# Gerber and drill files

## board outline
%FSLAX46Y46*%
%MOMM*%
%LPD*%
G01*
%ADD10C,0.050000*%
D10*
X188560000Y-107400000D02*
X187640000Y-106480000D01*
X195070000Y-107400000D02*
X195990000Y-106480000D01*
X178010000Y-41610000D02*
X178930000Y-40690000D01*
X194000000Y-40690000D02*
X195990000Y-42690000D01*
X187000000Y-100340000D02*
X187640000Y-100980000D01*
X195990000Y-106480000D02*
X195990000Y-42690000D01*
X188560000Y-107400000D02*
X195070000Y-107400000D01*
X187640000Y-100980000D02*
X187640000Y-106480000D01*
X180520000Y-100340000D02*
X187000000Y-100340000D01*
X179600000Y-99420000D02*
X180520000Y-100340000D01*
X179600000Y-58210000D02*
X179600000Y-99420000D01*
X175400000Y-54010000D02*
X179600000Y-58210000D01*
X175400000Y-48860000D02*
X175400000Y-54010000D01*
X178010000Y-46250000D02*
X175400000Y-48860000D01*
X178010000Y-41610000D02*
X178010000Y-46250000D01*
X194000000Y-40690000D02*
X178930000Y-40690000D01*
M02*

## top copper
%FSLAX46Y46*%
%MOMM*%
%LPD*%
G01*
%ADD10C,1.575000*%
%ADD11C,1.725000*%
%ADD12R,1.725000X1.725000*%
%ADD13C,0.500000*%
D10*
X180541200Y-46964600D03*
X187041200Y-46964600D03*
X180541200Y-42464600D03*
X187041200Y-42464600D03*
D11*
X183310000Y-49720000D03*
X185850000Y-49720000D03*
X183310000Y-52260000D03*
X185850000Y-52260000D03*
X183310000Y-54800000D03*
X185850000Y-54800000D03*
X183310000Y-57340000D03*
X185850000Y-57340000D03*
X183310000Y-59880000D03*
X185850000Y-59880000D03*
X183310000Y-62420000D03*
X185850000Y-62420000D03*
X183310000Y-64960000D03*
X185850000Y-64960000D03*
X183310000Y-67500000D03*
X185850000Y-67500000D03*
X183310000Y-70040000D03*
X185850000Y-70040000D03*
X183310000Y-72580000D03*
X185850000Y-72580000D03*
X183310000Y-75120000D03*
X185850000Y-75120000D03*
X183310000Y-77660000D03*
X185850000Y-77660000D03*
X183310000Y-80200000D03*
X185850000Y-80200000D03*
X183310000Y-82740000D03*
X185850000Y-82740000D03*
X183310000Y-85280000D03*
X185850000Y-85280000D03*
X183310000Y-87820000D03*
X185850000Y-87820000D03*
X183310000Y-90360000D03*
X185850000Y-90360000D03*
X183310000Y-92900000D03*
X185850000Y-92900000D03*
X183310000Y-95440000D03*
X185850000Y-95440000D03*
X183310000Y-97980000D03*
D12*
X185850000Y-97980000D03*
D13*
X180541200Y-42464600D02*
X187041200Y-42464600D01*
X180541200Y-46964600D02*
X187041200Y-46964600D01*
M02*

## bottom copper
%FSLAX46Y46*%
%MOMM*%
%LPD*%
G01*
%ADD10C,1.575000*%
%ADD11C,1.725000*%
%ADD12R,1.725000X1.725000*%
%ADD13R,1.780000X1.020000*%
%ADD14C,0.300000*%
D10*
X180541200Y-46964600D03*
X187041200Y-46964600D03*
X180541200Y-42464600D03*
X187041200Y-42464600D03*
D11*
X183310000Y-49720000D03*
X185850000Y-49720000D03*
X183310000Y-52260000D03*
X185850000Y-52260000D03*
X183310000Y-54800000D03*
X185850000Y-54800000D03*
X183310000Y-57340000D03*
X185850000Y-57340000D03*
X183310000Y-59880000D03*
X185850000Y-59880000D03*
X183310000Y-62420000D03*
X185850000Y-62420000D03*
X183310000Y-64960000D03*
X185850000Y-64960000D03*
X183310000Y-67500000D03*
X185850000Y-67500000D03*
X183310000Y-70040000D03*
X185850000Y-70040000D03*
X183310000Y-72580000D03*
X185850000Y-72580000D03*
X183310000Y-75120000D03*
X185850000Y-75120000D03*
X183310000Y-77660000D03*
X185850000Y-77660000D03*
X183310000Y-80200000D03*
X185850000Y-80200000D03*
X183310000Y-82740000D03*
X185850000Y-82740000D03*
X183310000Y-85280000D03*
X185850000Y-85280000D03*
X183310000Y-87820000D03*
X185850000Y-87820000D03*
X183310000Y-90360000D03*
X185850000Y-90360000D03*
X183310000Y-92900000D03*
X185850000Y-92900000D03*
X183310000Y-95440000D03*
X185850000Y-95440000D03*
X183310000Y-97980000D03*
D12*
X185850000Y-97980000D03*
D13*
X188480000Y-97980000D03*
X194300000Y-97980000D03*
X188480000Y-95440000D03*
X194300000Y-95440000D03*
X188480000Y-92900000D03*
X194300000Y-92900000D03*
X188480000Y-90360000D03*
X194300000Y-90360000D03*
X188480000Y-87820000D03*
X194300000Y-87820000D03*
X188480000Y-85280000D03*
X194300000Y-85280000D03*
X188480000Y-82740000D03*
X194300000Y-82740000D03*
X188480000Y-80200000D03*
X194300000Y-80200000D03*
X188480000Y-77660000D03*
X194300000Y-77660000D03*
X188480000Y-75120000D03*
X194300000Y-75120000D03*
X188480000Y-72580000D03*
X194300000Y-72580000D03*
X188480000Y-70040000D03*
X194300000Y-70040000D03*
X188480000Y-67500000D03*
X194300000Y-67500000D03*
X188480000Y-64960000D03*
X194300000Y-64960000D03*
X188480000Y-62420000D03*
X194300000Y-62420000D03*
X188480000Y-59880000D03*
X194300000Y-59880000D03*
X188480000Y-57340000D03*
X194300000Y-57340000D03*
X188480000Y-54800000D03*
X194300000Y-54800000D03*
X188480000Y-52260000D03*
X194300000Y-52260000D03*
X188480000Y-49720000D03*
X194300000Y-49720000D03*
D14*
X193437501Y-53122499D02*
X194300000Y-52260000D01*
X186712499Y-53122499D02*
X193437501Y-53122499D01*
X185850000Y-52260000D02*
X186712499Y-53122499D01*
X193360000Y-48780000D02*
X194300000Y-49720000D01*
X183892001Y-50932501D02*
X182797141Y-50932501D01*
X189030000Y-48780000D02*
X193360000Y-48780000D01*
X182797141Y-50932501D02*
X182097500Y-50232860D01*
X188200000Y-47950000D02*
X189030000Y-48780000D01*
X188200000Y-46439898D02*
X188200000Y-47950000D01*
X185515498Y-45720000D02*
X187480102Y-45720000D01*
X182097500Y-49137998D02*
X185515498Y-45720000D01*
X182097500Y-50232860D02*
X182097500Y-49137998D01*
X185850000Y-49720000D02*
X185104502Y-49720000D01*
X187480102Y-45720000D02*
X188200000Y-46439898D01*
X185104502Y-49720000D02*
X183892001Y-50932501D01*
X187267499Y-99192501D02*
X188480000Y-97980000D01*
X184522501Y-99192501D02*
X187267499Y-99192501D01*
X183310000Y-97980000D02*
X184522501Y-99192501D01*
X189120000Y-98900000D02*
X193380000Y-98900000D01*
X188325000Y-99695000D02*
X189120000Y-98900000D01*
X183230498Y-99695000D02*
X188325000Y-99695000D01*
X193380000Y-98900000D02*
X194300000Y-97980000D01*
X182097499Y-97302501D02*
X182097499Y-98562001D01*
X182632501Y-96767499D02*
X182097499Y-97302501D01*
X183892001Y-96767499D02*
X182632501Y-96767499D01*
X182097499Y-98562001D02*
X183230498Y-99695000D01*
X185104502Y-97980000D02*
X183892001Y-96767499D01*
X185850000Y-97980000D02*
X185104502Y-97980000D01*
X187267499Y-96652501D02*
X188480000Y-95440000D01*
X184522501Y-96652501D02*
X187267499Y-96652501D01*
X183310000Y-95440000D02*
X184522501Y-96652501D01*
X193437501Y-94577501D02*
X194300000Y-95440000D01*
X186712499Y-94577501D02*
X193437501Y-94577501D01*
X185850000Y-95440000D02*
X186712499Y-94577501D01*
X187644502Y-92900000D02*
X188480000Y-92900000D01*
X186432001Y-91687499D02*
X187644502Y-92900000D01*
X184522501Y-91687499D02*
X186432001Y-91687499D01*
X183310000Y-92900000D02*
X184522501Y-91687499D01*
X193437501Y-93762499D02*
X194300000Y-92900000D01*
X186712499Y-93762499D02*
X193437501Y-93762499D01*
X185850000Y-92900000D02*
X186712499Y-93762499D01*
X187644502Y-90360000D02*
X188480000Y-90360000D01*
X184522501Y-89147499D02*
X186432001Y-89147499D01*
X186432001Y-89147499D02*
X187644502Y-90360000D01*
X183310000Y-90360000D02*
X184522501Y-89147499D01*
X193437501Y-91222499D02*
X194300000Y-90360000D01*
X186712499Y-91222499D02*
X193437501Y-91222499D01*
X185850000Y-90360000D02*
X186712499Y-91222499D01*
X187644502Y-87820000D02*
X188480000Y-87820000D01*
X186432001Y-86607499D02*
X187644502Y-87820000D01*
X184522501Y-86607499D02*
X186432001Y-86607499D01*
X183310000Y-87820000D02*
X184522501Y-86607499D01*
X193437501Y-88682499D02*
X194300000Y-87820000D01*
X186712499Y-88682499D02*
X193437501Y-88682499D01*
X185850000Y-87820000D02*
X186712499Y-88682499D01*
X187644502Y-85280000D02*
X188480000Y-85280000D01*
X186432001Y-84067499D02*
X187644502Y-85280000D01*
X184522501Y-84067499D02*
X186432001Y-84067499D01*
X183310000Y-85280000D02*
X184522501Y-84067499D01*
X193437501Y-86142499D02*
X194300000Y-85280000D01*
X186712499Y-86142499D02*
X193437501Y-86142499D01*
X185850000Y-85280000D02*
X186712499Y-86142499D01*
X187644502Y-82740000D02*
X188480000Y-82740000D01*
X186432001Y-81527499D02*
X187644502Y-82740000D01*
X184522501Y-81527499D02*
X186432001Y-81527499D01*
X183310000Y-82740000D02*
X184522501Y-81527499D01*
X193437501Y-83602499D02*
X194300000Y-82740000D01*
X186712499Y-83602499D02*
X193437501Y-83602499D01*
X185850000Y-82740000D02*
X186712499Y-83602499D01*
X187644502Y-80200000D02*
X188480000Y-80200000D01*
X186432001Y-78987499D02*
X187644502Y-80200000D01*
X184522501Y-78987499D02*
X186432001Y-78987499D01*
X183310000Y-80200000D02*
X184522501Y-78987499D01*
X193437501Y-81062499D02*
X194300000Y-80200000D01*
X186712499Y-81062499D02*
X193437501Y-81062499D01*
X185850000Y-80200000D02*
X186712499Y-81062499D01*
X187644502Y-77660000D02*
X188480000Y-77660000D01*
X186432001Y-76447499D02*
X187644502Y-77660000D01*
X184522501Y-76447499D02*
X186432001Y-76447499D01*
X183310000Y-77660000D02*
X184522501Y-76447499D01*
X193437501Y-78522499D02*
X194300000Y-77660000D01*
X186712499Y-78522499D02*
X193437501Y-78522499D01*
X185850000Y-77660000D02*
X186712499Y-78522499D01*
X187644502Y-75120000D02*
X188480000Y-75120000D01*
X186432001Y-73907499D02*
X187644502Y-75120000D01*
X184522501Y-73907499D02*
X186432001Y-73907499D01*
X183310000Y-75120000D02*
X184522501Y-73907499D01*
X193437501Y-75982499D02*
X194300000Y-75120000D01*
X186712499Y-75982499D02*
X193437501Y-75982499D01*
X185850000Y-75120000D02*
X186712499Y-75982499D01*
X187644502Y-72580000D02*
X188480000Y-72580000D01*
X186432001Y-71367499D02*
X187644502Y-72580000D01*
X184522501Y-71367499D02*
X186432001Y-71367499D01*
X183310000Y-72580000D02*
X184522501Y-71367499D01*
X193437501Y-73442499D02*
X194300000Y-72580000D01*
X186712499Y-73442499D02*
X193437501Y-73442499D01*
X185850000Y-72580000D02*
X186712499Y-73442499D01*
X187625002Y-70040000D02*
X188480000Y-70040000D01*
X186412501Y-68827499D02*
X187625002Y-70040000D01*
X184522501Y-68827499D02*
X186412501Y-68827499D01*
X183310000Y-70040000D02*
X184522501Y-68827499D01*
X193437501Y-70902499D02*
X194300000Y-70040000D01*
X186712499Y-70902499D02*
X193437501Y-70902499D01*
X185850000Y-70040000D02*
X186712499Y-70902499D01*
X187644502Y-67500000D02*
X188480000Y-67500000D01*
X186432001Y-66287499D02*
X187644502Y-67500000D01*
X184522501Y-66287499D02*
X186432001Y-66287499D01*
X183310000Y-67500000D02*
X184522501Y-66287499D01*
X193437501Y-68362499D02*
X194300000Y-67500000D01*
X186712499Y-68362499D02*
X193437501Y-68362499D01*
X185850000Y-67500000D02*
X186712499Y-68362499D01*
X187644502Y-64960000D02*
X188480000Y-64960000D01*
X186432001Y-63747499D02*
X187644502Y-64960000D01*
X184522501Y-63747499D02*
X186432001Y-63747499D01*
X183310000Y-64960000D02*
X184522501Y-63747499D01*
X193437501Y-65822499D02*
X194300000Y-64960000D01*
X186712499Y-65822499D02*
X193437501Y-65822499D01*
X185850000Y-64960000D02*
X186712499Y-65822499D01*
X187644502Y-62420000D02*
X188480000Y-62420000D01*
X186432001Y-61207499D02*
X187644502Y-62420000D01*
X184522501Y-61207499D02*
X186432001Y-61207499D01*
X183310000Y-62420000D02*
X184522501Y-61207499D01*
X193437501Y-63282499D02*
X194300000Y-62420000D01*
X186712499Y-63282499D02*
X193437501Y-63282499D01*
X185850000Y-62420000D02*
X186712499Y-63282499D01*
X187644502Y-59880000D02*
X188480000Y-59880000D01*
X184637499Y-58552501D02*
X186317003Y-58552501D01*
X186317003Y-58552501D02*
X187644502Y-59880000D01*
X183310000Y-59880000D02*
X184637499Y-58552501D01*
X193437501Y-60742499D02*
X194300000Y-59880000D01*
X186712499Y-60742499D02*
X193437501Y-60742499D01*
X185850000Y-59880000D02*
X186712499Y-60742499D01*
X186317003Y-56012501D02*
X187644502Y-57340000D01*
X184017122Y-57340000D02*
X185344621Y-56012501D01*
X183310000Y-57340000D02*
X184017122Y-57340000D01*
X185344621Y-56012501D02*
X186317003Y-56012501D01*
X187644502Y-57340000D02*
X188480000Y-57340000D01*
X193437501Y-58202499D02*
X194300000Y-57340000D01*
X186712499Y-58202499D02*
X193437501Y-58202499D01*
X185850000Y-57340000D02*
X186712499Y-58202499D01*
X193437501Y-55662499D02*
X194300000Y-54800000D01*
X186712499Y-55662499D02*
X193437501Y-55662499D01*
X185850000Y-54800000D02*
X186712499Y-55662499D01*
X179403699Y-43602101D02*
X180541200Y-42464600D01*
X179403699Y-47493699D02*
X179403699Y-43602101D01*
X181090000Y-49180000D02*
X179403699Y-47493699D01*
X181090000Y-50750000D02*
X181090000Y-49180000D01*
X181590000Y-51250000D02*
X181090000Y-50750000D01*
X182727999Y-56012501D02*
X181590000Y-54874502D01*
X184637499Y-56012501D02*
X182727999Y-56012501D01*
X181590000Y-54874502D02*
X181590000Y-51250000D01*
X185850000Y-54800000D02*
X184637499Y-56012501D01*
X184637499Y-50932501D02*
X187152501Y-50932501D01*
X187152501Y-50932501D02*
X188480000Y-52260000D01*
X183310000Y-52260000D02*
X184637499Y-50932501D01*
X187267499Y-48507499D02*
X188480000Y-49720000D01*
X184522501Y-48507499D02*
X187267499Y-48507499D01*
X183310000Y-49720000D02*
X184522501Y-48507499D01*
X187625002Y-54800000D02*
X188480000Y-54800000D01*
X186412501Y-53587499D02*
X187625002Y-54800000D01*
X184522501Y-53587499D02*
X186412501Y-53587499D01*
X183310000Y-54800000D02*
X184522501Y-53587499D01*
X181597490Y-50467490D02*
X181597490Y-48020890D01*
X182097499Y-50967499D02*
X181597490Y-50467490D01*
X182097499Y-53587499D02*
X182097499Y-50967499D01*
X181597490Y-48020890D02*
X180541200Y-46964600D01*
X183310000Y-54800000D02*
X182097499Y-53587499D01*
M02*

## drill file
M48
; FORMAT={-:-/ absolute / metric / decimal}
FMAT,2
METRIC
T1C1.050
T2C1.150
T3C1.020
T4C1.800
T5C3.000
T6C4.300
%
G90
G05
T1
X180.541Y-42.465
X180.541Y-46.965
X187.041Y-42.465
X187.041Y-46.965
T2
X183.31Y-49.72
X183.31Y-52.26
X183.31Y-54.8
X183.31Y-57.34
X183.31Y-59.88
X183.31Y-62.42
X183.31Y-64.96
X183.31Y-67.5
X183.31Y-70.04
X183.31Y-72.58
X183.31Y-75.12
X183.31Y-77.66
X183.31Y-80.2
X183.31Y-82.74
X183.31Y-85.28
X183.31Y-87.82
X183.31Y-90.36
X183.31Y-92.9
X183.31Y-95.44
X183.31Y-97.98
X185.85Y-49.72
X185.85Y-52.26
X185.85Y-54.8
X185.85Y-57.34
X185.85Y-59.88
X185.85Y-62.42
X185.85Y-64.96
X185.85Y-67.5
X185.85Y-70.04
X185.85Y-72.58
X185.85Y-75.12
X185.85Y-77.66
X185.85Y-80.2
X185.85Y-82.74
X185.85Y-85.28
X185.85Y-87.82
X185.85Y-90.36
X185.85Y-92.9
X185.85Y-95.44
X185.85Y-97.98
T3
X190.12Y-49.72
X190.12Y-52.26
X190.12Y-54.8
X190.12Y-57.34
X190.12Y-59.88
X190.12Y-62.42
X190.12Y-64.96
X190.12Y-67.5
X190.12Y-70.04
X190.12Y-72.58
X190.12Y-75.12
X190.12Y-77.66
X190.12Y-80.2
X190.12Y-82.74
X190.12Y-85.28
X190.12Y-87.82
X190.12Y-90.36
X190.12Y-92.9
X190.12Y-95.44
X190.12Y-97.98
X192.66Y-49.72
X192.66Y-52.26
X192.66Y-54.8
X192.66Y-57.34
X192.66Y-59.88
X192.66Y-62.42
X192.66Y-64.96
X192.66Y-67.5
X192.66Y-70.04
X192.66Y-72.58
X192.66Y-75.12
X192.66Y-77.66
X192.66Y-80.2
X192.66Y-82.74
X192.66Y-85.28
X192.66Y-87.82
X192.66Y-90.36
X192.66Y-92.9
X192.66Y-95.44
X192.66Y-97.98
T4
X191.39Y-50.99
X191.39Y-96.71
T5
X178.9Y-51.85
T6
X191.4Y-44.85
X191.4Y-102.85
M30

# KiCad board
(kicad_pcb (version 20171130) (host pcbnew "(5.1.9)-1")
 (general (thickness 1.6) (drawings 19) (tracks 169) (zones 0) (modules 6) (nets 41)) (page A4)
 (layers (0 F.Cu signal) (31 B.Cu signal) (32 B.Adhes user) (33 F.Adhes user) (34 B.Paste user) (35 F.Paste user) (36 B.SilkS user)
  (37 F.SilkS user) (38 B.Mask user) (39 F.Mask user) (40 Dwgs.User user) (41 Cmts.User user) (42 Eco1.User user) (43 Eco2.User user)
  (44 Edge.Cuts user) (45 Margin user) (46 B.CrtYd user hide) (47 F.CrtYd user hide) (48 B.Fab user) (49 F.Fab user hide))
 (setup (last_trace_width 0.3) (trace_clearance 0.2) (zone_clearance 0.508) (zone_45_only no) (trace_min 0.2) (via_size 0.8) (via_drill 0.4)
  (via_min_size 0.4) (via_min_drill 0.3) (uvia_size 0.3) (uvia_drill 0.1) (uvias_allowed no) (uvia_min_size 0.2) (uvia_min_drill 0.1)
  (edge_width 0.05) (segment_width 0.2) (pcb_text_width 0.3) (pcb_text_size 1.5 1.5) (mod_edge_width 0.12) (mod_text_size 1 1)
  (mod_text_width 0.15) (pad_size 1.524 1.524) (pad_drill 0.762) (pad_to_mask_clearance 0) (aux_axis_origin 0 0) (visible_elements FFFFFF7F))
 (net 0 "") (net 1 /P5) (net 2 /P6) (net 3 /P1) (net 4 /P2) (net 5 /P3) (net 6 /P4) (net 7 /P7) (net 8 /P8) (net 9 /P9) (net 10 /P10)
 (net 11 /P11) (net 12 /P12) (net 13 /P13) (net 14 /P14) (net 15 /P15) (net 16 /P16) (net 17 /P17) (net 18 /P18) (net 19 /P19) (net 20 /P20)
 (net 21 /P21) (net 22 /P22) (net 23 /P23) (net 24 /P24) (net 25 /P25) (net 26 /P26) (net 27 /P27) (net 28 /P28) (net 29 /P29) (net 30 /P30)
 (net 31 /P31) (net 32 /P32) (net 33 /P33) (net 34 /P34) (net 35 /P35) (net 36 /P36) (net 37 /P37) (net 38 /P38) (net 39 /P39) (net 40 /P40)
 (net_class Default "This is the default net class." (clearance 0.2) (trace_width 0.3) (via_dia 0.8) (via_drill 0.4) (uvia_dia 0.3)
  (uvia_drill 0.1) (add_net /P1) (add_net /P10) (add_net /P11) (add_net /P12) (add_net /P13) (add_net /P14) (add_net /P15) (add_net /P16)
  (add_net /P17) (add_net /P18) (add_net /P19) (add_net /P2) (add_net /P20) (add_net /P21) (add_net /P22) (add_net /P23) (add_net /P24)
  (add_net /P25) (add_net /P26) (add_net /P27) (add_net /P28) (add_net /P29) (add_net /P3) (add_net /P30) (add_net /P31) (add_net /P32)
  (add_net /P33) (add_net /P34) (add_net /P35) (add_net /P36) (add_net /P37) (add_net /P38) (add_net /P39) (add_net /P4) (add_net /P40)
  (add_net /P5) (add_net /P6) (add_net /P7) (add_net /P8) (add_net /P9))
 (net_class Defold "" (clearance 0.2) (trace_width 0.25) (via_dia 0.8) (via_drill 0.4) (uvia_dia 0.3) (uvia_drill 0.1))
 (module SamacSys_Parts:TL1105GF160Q (layer F.Cu) (at 183.7912 44.7146)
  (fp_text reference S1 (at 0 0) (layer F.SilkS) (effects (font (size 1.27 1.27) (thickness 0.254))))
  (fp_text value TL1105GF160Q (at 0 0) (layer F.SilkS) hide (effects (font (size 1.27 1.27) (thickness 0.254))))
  (pad 1 thru_hole circle (at -3.25 2.25) (size 1.575 1.575) (drill 1.05) (layers *.Cu *.Mask) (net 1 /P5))
  (pad 2 thru_hole circle (at 3.25 2.25) (size 1.575 1.575) (drill 1.05) (layers *.Cu *.Mask) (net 1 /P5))
  (pad 3 thru_hole circle (at -3.25 -2.25) (size 1.575 1.575) (drill 1.05) (layers *.Cu *.Mask) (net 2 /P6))
  (pad 4 thru_hole circle (at 3.25 -2.25) (size 1.575 1.575) (drill 1.05) (layers *.Cu *.Mask) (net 2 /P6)))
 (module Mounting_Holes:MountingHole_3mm (layer F.Cu) (at 178.9 51.85)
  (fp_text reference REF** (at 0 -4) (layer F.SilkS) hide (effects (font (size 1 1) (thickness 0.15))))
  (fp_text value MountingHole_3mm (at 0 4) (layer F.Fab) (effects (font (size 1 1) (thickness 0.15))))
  (pad 1 np_thru_hole circle (at 0 0) (size 3 3) (drill 3) (layers *.Cu *.Mask)))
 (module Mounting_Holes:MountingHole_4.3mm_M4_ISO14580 (layer F.Cu) (at 191.4 102.85)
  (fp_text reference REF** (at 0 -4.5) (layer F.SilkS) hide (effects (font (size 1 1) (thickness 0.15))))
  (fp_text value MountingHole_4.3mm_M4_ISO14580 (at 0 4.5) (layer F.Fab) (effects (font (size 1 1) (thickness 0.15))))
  (pad 1 np_thru_hole circle (at 0 0) (size 4.3 4.3) (drill 4.3) (layers *.Cu *.Mask)))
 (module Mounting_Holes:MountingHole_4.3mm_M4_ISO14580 (layer F.Cu) (at 191.4 44.85)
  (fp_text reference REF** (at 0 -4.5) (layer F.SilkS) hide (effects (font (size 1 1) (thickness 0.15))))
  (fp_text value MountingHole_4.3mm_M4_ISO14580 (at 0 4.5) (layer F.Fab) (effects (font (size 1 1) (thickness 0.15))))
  (pad 1 np_thru_hole circle (at 0 0) (size 4.3 4.3) (drill 4.3) (layers *.Cu *.Mask)))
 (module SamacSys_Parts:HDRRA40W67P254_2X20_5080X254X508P (layer F.Cu) (at 185.85 97.98 270)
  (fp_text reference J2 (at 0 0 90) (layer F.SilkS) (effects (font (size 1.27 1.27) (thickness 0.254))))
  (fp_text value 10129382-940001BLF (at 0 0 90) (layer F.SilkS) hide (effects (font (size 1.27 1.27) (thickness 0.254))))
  (pad 40 thru_hole circle (at -48.26 2.54 270) (size 1.725 1.725) (drill 1.15) (layers *.Cu *.Mask) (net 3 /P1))
  (pad 39 thru_hole circle (at -48.26 0 270) (size 1.725 1.725) (drill 1.15) (layers *.Cu *.Mask) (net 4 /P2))
  (pad 38 thru_hole circle (at -45.72 2.54 270) (size 1.725 1.725) (drill 1.15) (layers *.Cu *.Mask) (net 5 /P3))
  (pad 37 thru_hole circle (at -45.72 0 270) (size 1.725 1.725) (drill 1.15) (layers *.Cu *.Mask) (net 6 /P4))
  (pad 36 thru_hole circle (at -43.18 2.54 270) (size 1.725 1.725) (drill 1.15) (layers *.Cu *.Mask) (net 1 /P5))
  (pad 35 thru_hole circle (at -43.18 0 270) (size 1.725 1.725) (drill 1.15) (layers *.Cu *.Mask) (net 2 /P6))
  (pad 34 thru_hole circle (at -40.64 2.54 270) (size 1.725 1.725) (drill 1.15) (layers *.Cu *.Mask) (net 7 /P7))
  (pad 33 thru_hole circle (at -40.64 0 270) (size 1.725 1.725) (drill 1.15) (layers *.Cu *.Mask) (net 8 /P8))
  (pad 32 thru_hole circle (at -38.1 2.54 270) (size 1.725 1.725) (drill 1.15) (layers *.Cu *.Mask) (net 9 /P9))
  (pad 31 thru_hole circle (at -38.1 0 270) (size 1.725 1.725) (drill 1.15) (layers *.Cu *.Mask) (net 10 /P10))
  (pad 30 thru_hole circle (at -35.56 2.54 270) (size 1.725 1.725) (drill 1.15) (layers *.Cu *.Mask) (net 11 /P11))
  (pad 29 thru_hole circle (at -35.56 0 270) (size 1.725 1.725) (drill 1.15) (layers *.Cu *.Mask) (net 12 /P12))
  (pad 28 thru_hole circle (at -33.02 2.54 270) (size 1.725 1.725) (drill 1.15) (layers *.Cu *.Mask) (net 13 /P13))
  (pad 27 thru_hole circle (at -33.02 0 270) (size 1.725 1.725) (drill 1.15) (layers *.Cu *.Mask) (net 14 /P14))
  (pad 26 thru_hole circle (at -30.48 2.54 270) (size 1.725 1.725) (drill 1.15) (layers *.Cu *.Mask) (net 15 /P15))
  (pad 25 thru_hole circle (at -30.48 0 270) (size 1.725 1.725) (drill 1.15) (layers *.Cu *.Mask) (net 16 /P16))
  (pad 24 thru_hole circle (at -27.94 2.54 270) (size 1.725 1.725) (drill 1.15) (layers *.Cu *.Mask) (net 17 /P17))
  (pad 23 thru_hole circle (at -27.94 0 270) (size 1.725 1.725) (drill 1.15) (layers *.Cu *.Mask) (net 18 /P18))
  (pad 22 thru_hole circle (at -25.4 2.54 270) (size 1.725 1.725) (drill 1.15) (layers *.Cu *.Mask) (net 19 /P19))
  (pad 21 thru_hole circle (at -25.4 0 270) (size 1.725 1.725) (drill 1.15) (layers *.Cu *.Mask) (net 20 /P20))
  (pad 20 thru_hole circle (at -22.86 2.54 270) (size 1.725 1.725) (drill 1.15) (layers *.Cu *.Mask) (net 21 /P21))
  (pad 19 thru_hole circle (at -22.86 0 270) (size 1.725 1.725) (drill 1.15) (layers *.Cu *.Mask) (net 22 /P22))
  (pad 18 thru_hole circle (at -20.32 2.54 270) (size 1.725 1.725) (drill 1.15) (layers *.Cu *.Mask) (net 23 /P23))
  (pad 17 thru_hole circle (at -20.32 0 270) (size 1.725 1.725) (drill 1.15) (layers *.Cu *.Mask) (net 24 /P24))
  (pad 16 thru_hole circle (at -17.78 2.54 270) (size 1.725 1.725) (drill 1.15) (layers *.Cu *.Mask) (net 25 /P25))
  (pad 15 thru_hole circle (at -17.78 0 270) (size 1.725 1.725) (drill 1.15) (layers *.Cu *.Mask) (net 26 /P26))
  (pad 14 thru_hole circle (at -15.24 2.54 270) (size 1.725 1.725) (drill 1.15) (layers *.Cu *.Mask) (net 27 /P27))
  (pad 13 thru_hole circle (at -15.24 0 270) (size 1.725 1.725) (drill 1.15) (layers *.Cu *.Mask) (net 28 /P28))
  (pad 12 thru_hole circle (at -12.7 2.54 270) (size 1.725 1.725) (drill 1.15) (layers *.Cu *.Mask) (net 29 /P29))
  (pad 11 thru_hole circle (at -12.7 0 270) (size 1.725 1.725) (drill 1.15) (layers *.Cu *.Mask) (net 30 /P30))
  (pad 10 thru_hole circle (at -10.16 2.54 270) (size 1.725 1.725) (drill 1.15) (layers *.Cu *.Mask) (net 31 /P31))
  (pad 9 thru_hole circle (at -10.16 0 270) (size 1.725 1.725) (drill 1.15) (layers *.Cu *.Mask) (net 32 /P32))
  (pad 8 thru_hole circle (at -7.62 2.54 270) (size 1.725 1.725) (drill 1.15) (layers *.Cu *.Mask) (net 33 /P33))
  (pad 7 thru_hole circle (at -7.62 0 270) (size 1.725 1.725) (drill 1.15) (layers *.Cu *.Mask) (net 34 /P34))
  (pad 6 thru_hole circle (at -5.08 2.54 270) (size 1.725 1.725) (drill 1.15) (layers *.Cu *.Mask) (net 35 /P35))
  (pad 5 thru_hole circle (at -5.08 0 270) (size 1.725 1.725) (drill 1.15) (layers *.Cu *.Mask) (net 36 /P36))
  (pad 4 thru_hole circle (at -2.54 2.54 270) (size 1.725 1.725) (drill 1.15) (layers *.Cu *.Mask) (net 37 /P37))
  (pad 3 thru_hole circle (at -2.54 0 270) (size 1.725 1.725) (drill 1.15) (layers *.Cu *.Mask) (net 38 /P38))
  (pad 2 thru_hole circle (at 0 2.54 270) (size 1.725 1.725) (drill 1.15) (layers *.Cu *.Mask) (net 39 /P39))
  (pad 1 thru_hole rect (at 0 0 270) (size 1.725 1.725) (drill 1.15) (layers *.Cu *.Mask) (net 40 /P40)))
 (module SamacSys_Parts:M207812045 (layer B.Cu) (at 191.39 73.85 270)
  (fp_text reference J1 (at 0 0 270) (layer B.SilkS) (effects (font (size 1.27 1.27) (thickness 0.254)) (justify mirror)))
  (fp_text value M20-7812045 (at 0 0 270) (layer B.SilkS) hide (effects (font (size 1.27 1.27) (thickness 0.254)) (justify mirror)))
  (pad MH2 np_thru_hole circle (at 22.86 0 270) (size 1.8 0) (drill 1.8) (layers *.Cu *.Mask))
  (pad MH1 np_thru_hole circle (at -22.86 0 270) (size 1.8 0) (drill 1.8) (layers *.Cu *.Mask))
  (pad 80 np_thru_hole circle (at 24.13 1.27 270) (size 1.02 0) (drill 1.02) (layers *.Cu *.Mask))
  (pad 79 np_thru_hole circle (at 24.13 -1.27 270) (size 1.02 0) (drill 1.02) (layers *.Cu *.Mask))
  (pad 78 np_thru_hole circle (at 21.59 1.27 270) (size 1.02 0) (drill 1.02) (layers *.Cu *.Mask))
  (pad 77 np_thru_hole circle (at 21.59 -1.27 270) (size 1.02 0) (drill 1.02) (layers *.Cu *.Mask))
  (pad 76 np_thru_hole circle (at 19.05 1.27 270) (size 1.02 0) (drill 1.02) (layers *.Cu *.Mask))
  (pad 75 np_thru_hole circle (at 19.05 -1.27 270) (size 1.02 0) (drill 1.02) (layers *.Cu *.Mask))
  (pad 74 np_thru_hole circle (at 16.51 1.27 270) (size 1.02 0) (drill 1.02) (layers *.Cu *.Mask))
  (pad 73 np_thru_hole circle (at 16.51 -1.27 270) (size 1.02 0) (drill 1.02) (layers *.Cu *.Mask))
  (pad 72 np_thru_hole circle (at 13.97 1.27 270) (size 1.02 0) (drill 1.02) (layers *.Cu *.Mask))
  (pad 71 np_thru_hole circle (at 13.97 -1.27 270) (size 1.02 0) (drill 1.02) (layers *.Cu *.Mask))
  (pad 70 np_thru_hole circle (at 11.43 1.27 270) (size 1.02 0) (drill 1.02) (layers *.Cu *.Mask))
  (pad 69 np_thru_hole circle (at 11.43 -1.27 270) (size 1.02 0) (drill 1.02) (layers *.Cu *.Mask))
  (pad 68 np_thru_hole circle (at 8.89 1.27 270) (size 1.02 0) (drill 1.02) (layers *.Cu *.Mask))
  (pad 67 np_thru_hole circle (at 8.89 -1.27 270) (size 1.02 0) (drill 1.02) (layers *.Cu *.Mask))
  (pad 66 np_thru_hole circle (at 6.35 1.27 270) (size 1.02 0) (drill 1.02) (layers *.Cu *.Mask))
  (pad 65 np_thru_hole circle (at 6.35 -1.27 270) (size 1.02 0) (drill 1.02) (layers *.Cu *.Mask))
  (pad 64 np_thru_hole circle (at 3.81 1.27 270) (size 1.02 0) (drill 1.02) (layers *.Cu *.Mask))
  (pad 63 np_thru_hole circle (at 3.81 -1.27 270) (size 1.02 0) (drill 1.02) (layers *.Cu *.Mask))
  (pad 62 np_thru_hole circle (at 1.27 1.27 270) (size 1.02 0) (drill 1.02) (layers *.Cu *.Mask))
  (pad 61 np_thru_hole circle (at 1.27 -1.27 270) (size 1.02 0) (drill 1.02) (layers *.Cu *.Mask))
  (pad 60 np_thru_hole circle (at -1.27 1.27 270) (size 1.02 0) (drill 1.02) (layers *.Cu *.Mask))
  (pad 59 np_thru_hole circle (at -1.27 -1.27 270) (size 1.02 0) (drill 1.02) (layers *.Cu *.Mask))
  (pad 58 np_thru_hole circle (at -3.81 1.27 270) (size 1.02 0) (drill 1.02) (layers *.Cu *.Mask))
  (pad 57 np_thru_hole circle (at -3.81 -1.27 270) (size 1.02 0) (drill 1.02) (layers *.Cu *.Mask))
  (pad 56 np_thru_hole circle (at -6.35 1.27 270) (size 1.02 0) (drill 1.02) (layers *.Cu *.Mask))
  (pad 55 np_thru_hole circle (at -6.35 -1.27 270) (size 1.02 0) (drill 1.02) (layers *.Cu *.Mask))
  (pad 54 np_thru_hole circle (at -8.89 1.27 270) (size 1.02 0) (drill 1.02) (layers *.Cu *.Mask))
  (pad 53 np_thru_hole circle (at -8.89 -1.27 270) (size 1.02 0) (drill 1.02) (layers *.Cu *.Mask))
  (pad 52 np_thru_hole circle (at -11.43 1.27 270) (size 1.02 0) (drill 1.02) (layers *.Cu *.Mask))
  (pad 51 np_thru_hole circle (at -11.43 -1.27 270) (size 1.02 0) (drill 1.02) (layers *.Cu *.Mask))
  (pad 50 np_thru_hole circle (at -13.97 1.27 270) (size 1.02 0) (drill 1.02) (layers *.Cu *.Mask))
  (pad 49 np_thru_hole circle (at -13.97 -1.27 270) (size 1.02 0) (drill 1.02) (layers *.Cu *.Mask))
  (pad 48 np_thru_hole circle (at -16.51 1.27 270) (size 1.02 0) (drill 1.02) (layers *.Cu *.Mask))
  (pad 47 np_thru_hole circle (at -16.51 -1.27 270) (size 1.02 0) (drill 1.02) (layers *.Cu *.Mask))
  (pad 46 np_thru_hole circle (at -19.05 1.27 270) (size 1.02 0) (drill 1.02) (layers *.Cu *.Mask))
  (pad 45 np_thru_hole circle (at -19.05 -1.27 270) (size 1.02 0) (drill 1.02) (layers *.Cu *.Mask))
  (pad 44 np_thru_hole circle (at -21.59 1.27 270) (size 1.02 0) (drill 1.02) (layers *.Cu *.Mask))
  (pad 43 np_thru_hole circle (at -21.59 -1.27 270) (size 1.02 0) (drill 1.02) (layers *.Cu *.Mask))
  (pad 42 np_thru_hole circle (at -24.13 1.27 270) (size 1.02 0) (drill 1.02) (layers *.Cu *.Mask))
  (pad 41 np_thru_hole circle (at -24.13 -1.27 270) (size 1.02 0) (drill 1.02) (layers *.Cu *.Mask))
  (pad 40 smd rect (at 24.13 2.91 270) (size 1.02 1.78) (layers B.Cu B.Paste B.Mask) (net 39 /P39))
  (pad 39 smd rect (at 24.13 -2.91 270) (size 1.02 1.78) (layers B.Cu B.Paste B.Mask) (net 40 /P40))
  (pad 38 smd rect (at 21.59 2.91 270) (size 1.02 1.78) (layers B.Cu B.Paste B.Mask) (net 37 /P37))
  (pad 37 smd rect (at 21.59 -2.91 270) (size 1.02 1.78) (layers B.Cu B.Paste B.Mask) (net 38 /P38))
  (pad 36 smd rect (at 19.05 2.91 270) (size 1.02 1.78) (layers B.Cu B.Paste B.Mask) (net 35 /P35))
  (pad 35 smd rect (at 19.05 -2.91 270) (size 1.02 1.78) (layers B.Cu B.Paste B.Mask) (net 36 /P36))
  (pad 34 smd rect (at 16.51 2.91 270) (size 1.02 1.78) (layers B.Cu B.Paste B.Mask) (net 33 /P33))
  (pad 33 smd rect (at 16.51 -2.91 270) (size 1.02 1.78) (layers B.Cu B.Paste B.Mask) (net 34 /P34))
  (pad 32 smd rect (at 13.97 2.91 270) (size 1.02 1.78) (layers B.Cu B.Paste B.Mask) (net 31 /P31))
  (pad 31 smd rect (at 13.97 -2.91 270) (size 1.02 1.78) (layers B.Cu B.Paste B.Mask) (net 32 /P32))
  (pad 30 smd rect (at 11.43 2.91 270) (size 1.02 1.78) (layers B.Cu B.Paste B.Mask) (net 29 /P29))
  (pad 29 smd rect (at 11.43 -2.91 270) (size 1.02 1.78) (layers B.Cu B.Paste B.Mask) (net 30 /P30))
  (pad 28 smd rect (at 8.89 2.91 270) (size 1.02 1.78) (layers B.Cu B.Paste B.Mask) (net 27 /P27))
  (pad 27 smd rect (at 8.89 -2.91 270) (size 1.02 1.78) (layers B.Cu B.Paste B.Mask) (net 28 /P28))
  (pad 26 smd rect (at 6.35 2.91 270) (size 1.02 1.78) (layers B.Cu B.Paste B.Mask) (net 25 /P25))
  (pad 25 smd rect (at 6.35 -2.91 270) (size 1.02 1.78) (layers B.Cu B.Paste B.Mask) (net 26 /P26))
  (pad 24 smd rect (at 3.81 2.91 270) (size 1.02 1.78) (layers B.Cu B.Paste B.Mask) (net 23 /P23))
  (pad 23 smd rect (at 3.81 -2.91 270) (size 1.02 1.78) (layers B.Cu B.Paste B.Mask) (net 24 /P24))
  (pad 22 smd rect (at 1.27 2.91 270) (size 1.02 1.78) (layers B.Cu B.Paste B.Mask) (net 21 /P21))
  (pad 21 smd rect (at 1.27 -2.91 270) (size 1.02 1.78) (layers B.Cu B.Paste B.Mask) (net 22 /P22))
  (pad 20 smd rect (at -1.27 2.91 270) (size 1.02 1.78) (layers B.Cu B.Paste B.Mask) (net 19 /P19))
  (pad 19 smd rect (at -1.27 -2.91 270) (size 1.02 1.78) (layers B.Cu B.Paste B.Mask) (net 20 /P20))
  (pad 18 smd rect (at -3.81 2.91 270) (size 1.02 1.78) (layers B.Cu B.Paste B.Mask) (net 17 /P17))
  (pad 17 smd rect (at -3.81 -2.91 270) (size 1.02 1.78) (layers B.Cu B.Paste B.Mask) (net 18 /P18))
  (pad 16 smd rect (at -6.35 2.91 270) (size 1.02 1.78) (layers B.Cu B.Paste B.Mask) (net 15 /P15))
  (pad 15 smd rect (at -6.35 -2.91 270) (size 1.02 1.78) (layers B.Cu B.Paste B.Mask) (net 16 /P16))
  (pad 14 smd rect (at -8.89 2.91 270) (size 1.02 1.78) (layers B.Cu B.Paste B.Mask) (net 13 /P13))
  (pad 13 smd rect (at -8.89 -2.91 270) (size 1.02 1.78) (layers B.Cu B.Paste B.Mask) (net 14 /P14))
  (pad 12 smd rect (at -11.43 2.91 270) (size 1.02 1.78) (layers B.Cu B.Paste B.Mask) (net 11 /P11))
  (pad 11 smd rect (at -11.43 -2.91 270) (size 1.02 1.78) (layers B.Cu B.Paste B.Mask) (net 12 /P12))
  (pad 10 smd rect (at -13.97 2.91 270) (size 1.02 1.78) (layers B.Cu B.Paste B.Mask) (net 9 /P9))
  (pad 9 smd rect (at -13.97 -2.91 270) (size 1.02 1.78) (layers B.Cu B.Paste B.Mask) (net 10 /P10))
  (pad 8 smd rect (at -16.51 2.91 270) (size 1.02 1.78) (layers B.Cu B.Paste B.Mask) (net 7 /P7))
  (pad 7 smd rect (at -16.51 -2.91 270) (size 1.02 1.78) (layers B.Cu B.Paste B.Mask) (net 8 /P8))
  (pad 6 smd rect (at -19.05 2.91 270) (size 1.02 1.78) (layers B.Cu B.Paste B.Mask) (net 1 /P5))
  (pad 5 smd rect (at -19.05 -2.91 270) (size 1.02 1.78) (layers B.Cu B.Paste B.Mask) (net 2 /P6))
  (pad 4 smd rect (at -21.59 2.91 270) (size 1.02 1.78) (layers B.Cu B.Paste B.Mask) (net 5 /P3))
  (pad 3 smd rect (at -21.59 -2.91 270) (size 1.02 1.78) (layers B.Cu B.Paste B.Mask) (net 6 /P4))
  (pad 2 smd rect (at -24.13 2.91 270) (size 1.02 1.78) (layers B.Cu B.Paste B.Mask) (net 3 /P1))
  (pad 1 smd rect (at -24.13 -2.91 270) (size 1.02 1.78) (layers B.Cu B.Paste B.Mask) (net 4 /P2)))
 (gr_line (start 188.56 107.4) (end 187.64 106.48) (layer Edge.Cuts) (width 0.05))
 (gr_line (start 195.07 107.4) (end 195.99 106.48) (layer Edge.Cuts) (width 0.05))
 (gr_line (start 178.01 41.61) (end 178.93 40.69) (layer Edge.Cuts) (width 0.05))
 (gr_line (start 194 40.69) (end 195.99 42.69) (layer Edge.Cuts) (width 0.05))
 (gr_line (start 187 100.34) (end 187.64 100.98) (layer Edge.Cuts) (width 0.05))
 (gr_line (start 195.99 106.48) (end 195.99 42.69) (layer Edge.Cuts) (width 0.05))
 (gr_line (start 188.56 107.4) (end 195.07 107.4) (layer Edge.Cuts) (width 0.05))
 (gr_line (start 187.64 100.98) (end 187.64 106.48) (layer Edge.Cuts) (width 0.05))
 (gr_line (start 180.52 100.34) (end 187 100.34) (layer Edge.Cuts) (width 0.05))
 (gr_line (start 179.6 99.42) (end 180.52 100.34) (layer Edge.Cuts) (width 0.05))
 (gr_line (start 179.6 58.21) (end 179.6 99.42) (layer Edge.Cuts) (width 0.05))
 (gr_line (start 175.4 54.01) (end 179.6 58.21) (layer Edge.Cuts) (width 0.05))
 (gr_line (start 175.4 48.86) (end 175.4 54.01) (layer Edge.Cuts) (width 0.05))
 (gr_line (start 178.01 46.25) (end 175.4 48.86) (layer Edge.Cuts) (width 0.05))
 (gr_line (start 178.01 41.61) (end 178.01 46.25) (layer Edge.Cuts) (width 0.05))
 (gr_line (start 194 40.69) (end 178.93 40.69) (layer Edge.Cuts) (width 0.05))
 (segment (start 193.437501 53.122499) (end 194.3 52.26) (width 0.3) (layer B.Cu) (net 6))
 (segment (start 186.712499 53.122499) (end 193.437501 53.122499) (width 0.3) (layer B.Cu) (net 6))
 (segment (start 185.85 52.26) (end 186.712499 53.122499) (width 0.3) (layer B.Cu) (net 6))
 (segment (start 193.36 48.78) (end 194.3 49.72) (width 0.3) (layer B.Cu) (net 4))
 (segment (start 183.892001 50.932501) (end 182.797141 50.932501) (width 0.3) (layer B.Cu) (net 4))
 (segment (start 189.03 48.78) (end 193.36 48.78) (width 0.3) (layer B.Cu) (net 4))
 (segment (start 182.797141 50.932501) (end 182.0975 50.23286) (width 0.3) (layer B.Cu) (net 4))
 (segment (start 188.2 47.95) (end 189.03 48.78) (width 0.3) (layer B.Cu) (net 4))
 (segment (start 188.2 46.439898) (end 188.2 47.95) (width 0.3) (layer B.Cu) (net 4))
 (segment (start 185.515498 45.72) (end 187.480102 45.72) (width 0.3) (layer B.Cu) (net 4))
 (segment (start 182.0975 49.137998) (end 185.515498 45.72) (width 0.3) (layer B.Cu) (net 4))
 (segment (start 182.0975 50.23286) (end 182.0975 49.137998) (width 0.3) (layer B.Cu) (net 4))
 (segment (start 185.85 49.72) (end 185.104502 49.72) (width 0.3) (layer B.Cu) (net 4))
 (segment (start 187.480102 45.72) (end 188.2 46.439898) (width 0.3) (layer B.Cu) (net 4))
 (segment (start 185.104502 49.72) (end 183.892001 50.932501) (width 0.3) (layer B.Cu) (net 4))
 (segment (start 187.267499 99.192501) (end 188.48 97.98) (width 0.3) (layer B.Cu) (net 39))
 (segment (start 184.522501 99.192501) (end 187.267499 99.192501) (width 0.3) (layer B.Cu) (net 39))
 (segment (start 183.31 97.98) (end 184.522501 99.192501) (width 0.3) (layer B.Cu) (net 39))
 (segment (start 189.12 98.9) (end 193.38 98.9) (width 0.3) (layer B.Cu) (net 40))
 (segment (start 188.325 99.695) (end 189.12 98.9) (width 0.3) (layer B.Cu) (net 40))
 (segment (start 183.230498 99.695) (end 188.325 99.695) (width 0.3) (layer B.Cu) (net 40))
 (segment (start 193.38 98.9) (end 194.3 97.98) (width 0.3) (layer B.Cu) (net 40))
 (segment (start 182.097499 97.302501) (end 182.097499 98.562001) (width 0.3) (layer B.Cu) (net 40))
 (segment (start 182.632501 96.767499) (end 182.097499 97.302501) (width 0.3) (layer B.Cu) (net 40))
 (segment (start 183.892001 96.767499) (end 182.632501 96.767499) (width 0.3) (layer B.Cu) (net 40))
 (segment (start 182.097499 98.562001) (end 183.230498 99.695) (width 0.3) (layer B.Cu) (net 40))
 (segment (start 185.104502 97.98) (end 183.892001 96.767499) (width 0.3) (layer B.Cu) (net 40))
 (segment (start 185.85 97.98) (end 185.104502 97.98) (width 0.3) (layer B.Cu) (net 40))
 (segment (start 187.267499 96.652501) (end 188.48 95.44) (width 0.3) (layer B.Cu) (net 37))
 (segment (start 184.522501 96.652501) (end 187.267499 96.652501) (width 0.3) (layer B.Cu) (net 37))
 (segment (start 183.31 95.44) (end 184.522501 96.652501) (width 0.3) (layer B.Cu) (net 37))
 (segment (start 193.437501 94.577501) (end 194.3 95.44) (width 0.3) (layer B.Cu) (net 38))
 (segment (start 186.712499 94.577501) (end 193.437501 94.577501) (width 0.3) (layer B.Cu) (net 38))
 (segment (start 185.85 95.44) (end 186.712499 94.577501) (width 0.3) (layer B.Cu) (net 38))
 (segment (start 187.644502 92.9) (end 188.48 92.9) (width 0.3) (layer B.Cu) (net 35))
 (segment (start 186.432001 91.687499) (end 187.644502 92.9) (width 0.3) (layer B.Cu) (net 35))
 (segment (start 184.522501 91.687499) (end 186.432001 91.687499) (width 0.3) (layer B.Cu) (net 35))
 (segment (start 183.31 92.9) (end 184.522501 91.687499) (width 0.3) (layer B.Cu) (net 35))
 (segment (start 193.437501 93.762499) (end 194.3 92.9) (width 0.3) (layer B.Cu) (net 36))
 (segment (start 186.712499 93.762499) (end 193.437501 93.762499) (width 0.3) (layer B.Cu) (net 36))
 (segment (start 185.85 92.9) (end 186.712499 93.762499) (width 0.3) (layer B.Cu) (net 36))
 (segment (start 187.644502 90.36) (end 188.48 90.36) (width 0.3) (layer B.Cu) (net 33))
 (segment (start 184.522501 89.147499) (end 186.432001 89.147499) (width 0.3) (layer B.Cu) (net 33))
 (segment (start 186.432001 89.147499) (end 187.644502 90.36) (width 0.3) (layer B.Cu) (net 33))
 (segment (start 183.31 90.36) (end 184.522501 89.147499) (width 0.3) (layer B.Cu) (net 33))
 (segment (start 193.437501 91.222499) (end 194.3 90.36) (width 0.3) (layer B.Cu) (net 34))
 (segment (start 186.712499 91.222499) (end 193.437501 91.222499) (width 0.3) (layer B.Cu) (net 34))
 (segment (start 185.85 90.36) (end 186.712499 91.222499) (width 0.3) (layer B.Cu) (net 34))
 (segment (start 187.644502 87.82) (end 188.48 87.82) (width 0.3) (layer B.Cu) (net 31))
 (segment (start 186.432001 86.607499) (end 187.644502 87.82) (width 0.3) (layer B.Cu) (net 31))
 (segment (start 184.522501 86.607499) (end 186.432001 86.607499) (width 0.3) (layer B.Cu) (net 31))
 (segment (start 183.31 87.82) (end 184.522501 86.607499) (width 0.3) (layer B.Cu) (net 31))
 (segment (start 193.437501 88.682499) (end 194.3 87.82) (width 0.3) (layer B.Cu) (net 32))
 (segment (start 186.712499 88.682499) (end 193.437501 88.682499) (width 0.3) (layer B.Cu) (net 32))
 (segment (start 185.85 87.82) (end 186.712499 88.682499) (width 0.3) (layer B.Cu) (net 32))
 (segment (start 187.644502 85.28) (end 188.48 85.28) (width 0.3) (layer B.Cu) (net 29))
 (segment (start 186.432001 84.067499) (end 187.644502 85.28) (width 0.3) (layer B.Cu) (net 29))
 (segment (start 184.522501 84.067499) (end 186.432001 84.067499) (width 0.3) (layer B.Cu) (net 29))
 (segment (start 183.31 85.28) (end 184.522501 84.067499) (width 0.3) (layer B.Cu) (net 29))
 (segment (start 193.437501 86.142499) (end 194.3 85.28) (width 0.3) (layer B.Cu) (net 30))
 (segment (start 186.712499 86.142499) (end 193.437501 86.142499) (width 0.3) (layer B.Cu) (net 30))
 (segment (start 185.85 85.28) (end 186.712499 86.142499) (width 0.3) (layer B.Cu) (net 30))
 (segment (start 187.644502 82.74) (end 188.48 82.74) (width 0.3) (layer B.Cu) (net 27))
 (segment (start 186.432001 81.527499) (end 187.644502 82.74) (width 0.3) (layer B.Cu) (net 27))
 (segment (start 184.522501 81.527499) (end 186.432001 81.527499) (width 0.3) (layer B.Cu) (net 27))
 (segment (start 183.31 82.74) (end 184.522501 81.527499) (width 0.3) (layer B.Cu) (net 27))
 (segment (start 193.437501 83.602499) (end 194.3 82.74) (width 0.3) (layer B.Cu) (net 28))
 (segment (start 186.712499 83.602499) (end 193.437501 83.602499) (width 0.3) (layer B.Cu) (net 28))
 (segment (start 185.85 82.74) (end 186.712499 83.602499) (width 0.3) (layer B.Cu) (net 28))
 (segment (start 187.644502 80.2) (end 188.48 80.2) (width 0.3) (layer B.Cu) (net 25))
 (segment (start 186.432001 78.987499) (end 187.644502 80.2) (width 0.3) (layer B.Cu) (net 25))
 (segment (start 184.522501 78.987499) (end 186.432001 78.987499) (width 0.3) (layer B.Cu) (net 25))
 (segment (start 183.31 80.2) (end 184.522501 78.987499) (width 0.3) (layer B.Cu) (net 25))
 (segment (start 193.437501 81.062499) (end 194.3 80.2) (width 0.3) (layer B.Cu) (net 26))
 (segment (start 186.712499 81.062499) (end 193.437501 81.062499) (width 0.3) (layer B.Cu) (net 26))
 (segment (start 185.85 80.2) (end 186.712499 81.062499) (width 0.3) (layer B.Cu) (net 26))
 (segment (start 187.644502 77.66) (end 188.48 77.66) (width 0.3) (layer B.Cu) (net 23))
 (segment (start 186.432001 76.447499) (end 187.644502 77.66) (width 0.3) (layer B.Cu) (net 23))
 (segment (start 184.522501 76.447499) (end 186.432001 76.447499) (width 0.3) (layer B.Cu) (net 23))
 (segment (start 183.31 77.66) (end 184.522501 76.447499) (width 0.3) (layer B.Cu) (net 23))
 (segment (start 193.437501 78.522499) (end 194.3 77.66) (width 0.3) (layer B.Cu) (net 24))
 (segment (start 186.712499 78.522499) (end 193.437501 78.522499) (width 0.3) (layer B.Cu) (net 24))
 (segment (start 185.85 77.66) (end 186.712499 78.522499) (width 0.3) (layer B.Cu) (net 24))
 (segment (start 187.644502 75.12) (end 188.48 75.12) (width 0.3) (layer B.Cu) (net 21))
 (segment (start 186.432001 73.907499) (end 187.644502 75.12) (width 0.3) (layer B.Cu) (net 21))
 (segment (start 184.522501 73.907499) (end 186.432001 73.907499) (width 0.3) (layer B.Cu) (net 21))
 (segment (start 183.31 75.12) (end 184.522501 73.907499) (width 0.3) (layer B.Cu) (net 21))
 (segment (start 193.437501 75.982499) (end 194.3 75.12) (width 0.3) (layer B.Cu) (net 22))
 (segment (start 186.712499 75.982499) (end 193.437501 75.982499) (width 0.3) (layer B.Cu) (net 22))
 (segment (start 185.85 75.12) (end 186.712499 75.982499) (width 0.3) (layer B.Cu) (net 22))
 (segment (start 187.644502 72.58) (end 188.48 72.58) (width 0.3) (layer B.Cu) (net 19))
 (segment (start 186.432001 71.367499) (end 187.644502 72.58) (width 0.3) (layer B.Cu) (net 19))
 (segment (start 184.522501 71.367499) (end 186.432001 71.367499) (width 0.3) (layer B.Cu) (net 19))
 (segment (start 183.31 72.58) (end 184.522501 71.367499) (width 0.3) (layer B.Cu) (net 19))
 (segment (start 193.437501 73.442499) (end 194.3 72.58) (width 0.3) (layer B.Cu) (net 20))
 (segment (start 186.712499 73.442499) (end 193.437501 73.442499) (width 0.3) (layer B.Cu) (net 20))
 (segment (start 185.85 72.58) (end 186.712499 73.442499) (width 0.3) (layer B.Cu) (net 20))
 (segment (start 187.625002 70.04) (end 188.48 70.04) (width 0.3) (layer B.Cu) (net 17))
 (segment (start 186.412501 68.827499) (end 187.625002 70.04) (width 0.3) (layer B.Cu) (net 17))
 (segment (start 184.522501 68.827499) (end 186.412501 68.827499) (width 0.3) (layer B.Cu) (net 17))
 (segment (start 183.31 70.04) (end 184.522501 68.827499) (width 0.3) (layer B.Cu) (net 17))
 (segment (start 193.437501 70.902499) (end 194.3 70.04) (width 0.3) (layer B.Cu) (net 18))
 (segment (start 186.712499 70.902499) (end 193.437501 70.902499) (width 0.3) (layer B.Cu) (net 18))
 (segment (start 185.85 70.04) (end 186.712499 70.902499) (width 0.3) (layer B.Cu) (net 18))
 (segment (start 187.644502 67.5) (end 188.48 67.5) (width 0.3) (layer B.Cu) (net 15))
 (segment (start 186.432001 66.287499) (end 187.644502 67.5) (width 0.3) (layer B.Cu) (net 15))
 (segment (start 184.522501 66.287499) (end 186.432001 66.287499) (width 0.3) (layer B.Cu) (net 15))
 (segment (start 183.31 67.5) (end 184.522501 66.287499) (width 0.3) (layer B.Cu) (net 15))
 (segment (start 193.437501 68.362499) (end 194.3 67.5) (width 0.3) (layer B.Cu) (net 16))
 (segment (start 186.712499 68.362499) (end 193.437501 68.362499) (width 0.3) (layer B.Cu) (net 16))
 (segment (start 185.85 67.5) (end 186.712499 68.362499) (width 0.3) (layer B.Cu) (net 16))
 (segment (start 187.644502 64.96) (end 188.48 64.96) (width 0.3) (layer B.Cu) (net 13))
 (segment (start 186.432001 63.747499) (end 187.644502 64.96) (width 0.3) (layer B.Cu) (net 13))
 (segment (start 184.522501 63.747499) (end 186.432001 63.747499) (width 0.3) (layer B.Cu) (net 13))
 (segment (start 183.31 64.96) (end 184.522501 63.747499) (width 0.3) (layer B.Cu) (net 13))
 (segment (start 193.437501 65.822499) (end 194.3 64.96) (width 0.3) (layer B.Cu) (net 14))
 (segment (start 186.712499 65.822499) (end 193.437501 65.822499) (width 0.3) (layer B.Cu) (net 14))
 (segment (start 185.85 64.96) (end 186.712499 65.822499) (width 0.3) (layer B.Cu) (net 14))
 (segment (start 187.644502 62.42) (end 188.48 62.42) (width 0.3) (layer B.Cu) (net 11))
 (segment (start 186.432001 61.207499) (end 187.644502 62.42) (width 0.3) (layer B.Cu) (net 11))
 (segment (start 184.522501 61.207499) (end 186.432001 61.207499) (width 0.3) (layer B.Cu) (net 11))
 (segment (start 183.31 62.42) (end 184.522501 61.207499) (width 0.3) (layer B.Cu) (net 11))
 (segment (start 193.437501 63.282499) (end 194.3 62.42) (width 0.3) (layer B.Cu) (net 12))
 (segment (start 186.712499 63.282499) (end 193.437501 63.282499) (width 0.3) (layer B.Cu) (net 12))
 (segment (start 185.85 62.42) (end 186.712499 63.282499) (width 0.3) (layer B.Cu) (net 12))
 (segment (start 187.644502 59.88) (end 188.48 59.88) (width 0.3) (layer B.Cu) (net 9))
 (segment (start 184.637499 58.552501) (end 186.317003 58.552501) (width 0.3) (layer B.Cu) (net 9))
 (segment (start 186.317003 58.552501) (end 187.644502 59.88) (width 0.3) (layer B.Cu) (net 9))
 (segment (start 183.31 59.88) (end 184.637499 58.552501) (width 0.3) (layer B.Cu) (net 9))
 (segment (start 193.437501 60.742499) (end 194.3 59.88) (width 0.3) (layer B.Cu) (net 10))
 (segment (start 186.712499 60.742499) (end 193.437501 60.742499) (width 0.3) (layer B.Cu) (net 10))
 (segment (start 185.85 59.88) (end 186.712499 60.742499) (width 0.3) (layer B.Cu) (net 10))
 (segment (start 186.317003 56.012501) (end 187.644502 57.34) (width 0.3) (layer B.Cu) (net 7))
 (segment (start 184.017122 57.34) (end 185.344621 56.012501) (width 0.3) (layer B.Cu) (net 7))
 (segment (start 183.31 57.34) (end 184.017122 57.34) (width 0.3) (layer B.Cu) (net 7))
 (segment (start 185.344621 56.012501) (end 186.317003 56.012501) (width 0.3) (layer B.Cu) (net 7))
 (segment (start 187.644502 57.34) (end 188.48 57.34) (width 0.3) (layer B.Cu) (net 7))
 (segment (start 193.437501 58.202499) (end 194.3 57.34) (width 0.3) (layer B.Cu) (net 8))
 (segment (start 186.712499 58.202499) (end 193.437501 58.202499) (width 0.3) (layer B.Cu) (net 8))
 (segment (start 185.85 57.34) (end 186.712499 58.202499) (width 0.3) (layer B.Cu) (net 8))
 (segment (start 193.437501 55.662499) (end 194.3 54.8) (width 0.3) (layer B.Cu) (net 2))
 (segment (start 186.712499 55.662499) (end 193.437501 55.662499) (width 0.3) (layer B.Cu) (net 2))
 (segment (start 185.85 54.8) (end 186.712499 55.662499) (width 0.3) (layer B.Cu) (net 2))
 (segment (start 180.5412 42.4646) (end 187.0412 42.4646) (width 0.5) (layer F.Cu) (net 2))
 (segment (start 179.403699 43.602101) (end 180.5412 42.4646) (width 0.3) (layer B.Cu) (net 2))
 (segment (start 179.403699 47.493699) (end 179.403699 43.602101) (width 0.3) (layer B.Cu) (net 2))
 (segment (start 181.09 49.18) (end 179.403699 47.493699) (width 0.3) (layer B.Cu) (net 2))
 (segment (start 181.09 50.75) (end 181.09 49.18) (width 0.3) (layer B.Cu) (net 2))
 (segment (start 181.59 51.25) (end 181.09 50.75) (width 0.3) (layer B.Cu) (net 2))
 (segment (start 182.727999 56.012501) (end 181.59 54.874502) (width 0.3) (layer B.Cu) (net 2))
 (segment (start 184.637499 56.012501) (end 182.727999 56.012501) (width 0.3) (layer B.Cu) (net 2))
 (segment (start 181.59 54.874502) (end 181.59 51.25) (width 0.3) (layer B.Cu) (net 2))
 (segment (start 185.85 54.8) (end 184.637499 56.012501) (width 0.3) (layer B.Cu) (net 2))
 (segment (start 184.637499 50.932501) (end 187.152501 50.932501) (width 0.3) (layer B.Cu) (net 5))
 (segment (start 187.152501 50.932501) (end 188.48 52.26) (width 0.3) (layer B.Cu) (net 5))
 (segment (start 183.31 52.26) (end 184.637499 50.932501) (width 0.3) (layer B.Cu) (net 5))
 (segment (start 187.267499 48.507499) (end 188.48 49.72) (width 0.3) (layer B.Cu) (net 3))
 (segment (start 184.522501 48.507499) (end 187.267499 48.507499) (width 0.3) (layer B.Cu) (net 3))
 (segment (start 183.31 49.72) (end 184.522501 48.507499) (width 0.3) (layer B.Cu) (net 3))
 (segment (start 187.625002 54.8) (end 188.48 54.8) (width 0.3) (layer B.Cu) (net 1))
 (segment (start 186.412501 53.587499) (end 187.625002 54.8) (width 0.3) (layer B.Cu) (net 1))
 (segment (start 184.522501 53.587499) (end 186.412501 53.587499) (width 0.3) (layer B.Cu) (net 1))
 (segment (start 183.31 54.8) (end 184.522501 53.587499) (width 0.3) (layer B.Cu) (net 1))
 (segment (start 180.5412 46.9646) (end 187.0412 46.9646) (width 0.5) (layer F.Cu) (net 1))
 (segment (start 181.59749 50.46749) (end 181.59749 48.02089) (width 0.3) (layer B.Cu) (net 1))
 (segment (start 182.097499 50.967499) (end 181.59749 50.46749) (width 0.3) (layer B.Cu) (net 1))
 (segment (start 182.097499 53.587499) (end 182.097499 50.967499) (width 0.3) (layer B.Cu) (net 1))
 (segment (start 181.59749 48.02089) (end 180.5412 46.9646) (width 0.3) (layer B.Cu) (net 1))
 (segment (start 183.31 54.8) (end 182.097499 53.587499) (width 0.3) (layer B.Cu) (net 1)))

